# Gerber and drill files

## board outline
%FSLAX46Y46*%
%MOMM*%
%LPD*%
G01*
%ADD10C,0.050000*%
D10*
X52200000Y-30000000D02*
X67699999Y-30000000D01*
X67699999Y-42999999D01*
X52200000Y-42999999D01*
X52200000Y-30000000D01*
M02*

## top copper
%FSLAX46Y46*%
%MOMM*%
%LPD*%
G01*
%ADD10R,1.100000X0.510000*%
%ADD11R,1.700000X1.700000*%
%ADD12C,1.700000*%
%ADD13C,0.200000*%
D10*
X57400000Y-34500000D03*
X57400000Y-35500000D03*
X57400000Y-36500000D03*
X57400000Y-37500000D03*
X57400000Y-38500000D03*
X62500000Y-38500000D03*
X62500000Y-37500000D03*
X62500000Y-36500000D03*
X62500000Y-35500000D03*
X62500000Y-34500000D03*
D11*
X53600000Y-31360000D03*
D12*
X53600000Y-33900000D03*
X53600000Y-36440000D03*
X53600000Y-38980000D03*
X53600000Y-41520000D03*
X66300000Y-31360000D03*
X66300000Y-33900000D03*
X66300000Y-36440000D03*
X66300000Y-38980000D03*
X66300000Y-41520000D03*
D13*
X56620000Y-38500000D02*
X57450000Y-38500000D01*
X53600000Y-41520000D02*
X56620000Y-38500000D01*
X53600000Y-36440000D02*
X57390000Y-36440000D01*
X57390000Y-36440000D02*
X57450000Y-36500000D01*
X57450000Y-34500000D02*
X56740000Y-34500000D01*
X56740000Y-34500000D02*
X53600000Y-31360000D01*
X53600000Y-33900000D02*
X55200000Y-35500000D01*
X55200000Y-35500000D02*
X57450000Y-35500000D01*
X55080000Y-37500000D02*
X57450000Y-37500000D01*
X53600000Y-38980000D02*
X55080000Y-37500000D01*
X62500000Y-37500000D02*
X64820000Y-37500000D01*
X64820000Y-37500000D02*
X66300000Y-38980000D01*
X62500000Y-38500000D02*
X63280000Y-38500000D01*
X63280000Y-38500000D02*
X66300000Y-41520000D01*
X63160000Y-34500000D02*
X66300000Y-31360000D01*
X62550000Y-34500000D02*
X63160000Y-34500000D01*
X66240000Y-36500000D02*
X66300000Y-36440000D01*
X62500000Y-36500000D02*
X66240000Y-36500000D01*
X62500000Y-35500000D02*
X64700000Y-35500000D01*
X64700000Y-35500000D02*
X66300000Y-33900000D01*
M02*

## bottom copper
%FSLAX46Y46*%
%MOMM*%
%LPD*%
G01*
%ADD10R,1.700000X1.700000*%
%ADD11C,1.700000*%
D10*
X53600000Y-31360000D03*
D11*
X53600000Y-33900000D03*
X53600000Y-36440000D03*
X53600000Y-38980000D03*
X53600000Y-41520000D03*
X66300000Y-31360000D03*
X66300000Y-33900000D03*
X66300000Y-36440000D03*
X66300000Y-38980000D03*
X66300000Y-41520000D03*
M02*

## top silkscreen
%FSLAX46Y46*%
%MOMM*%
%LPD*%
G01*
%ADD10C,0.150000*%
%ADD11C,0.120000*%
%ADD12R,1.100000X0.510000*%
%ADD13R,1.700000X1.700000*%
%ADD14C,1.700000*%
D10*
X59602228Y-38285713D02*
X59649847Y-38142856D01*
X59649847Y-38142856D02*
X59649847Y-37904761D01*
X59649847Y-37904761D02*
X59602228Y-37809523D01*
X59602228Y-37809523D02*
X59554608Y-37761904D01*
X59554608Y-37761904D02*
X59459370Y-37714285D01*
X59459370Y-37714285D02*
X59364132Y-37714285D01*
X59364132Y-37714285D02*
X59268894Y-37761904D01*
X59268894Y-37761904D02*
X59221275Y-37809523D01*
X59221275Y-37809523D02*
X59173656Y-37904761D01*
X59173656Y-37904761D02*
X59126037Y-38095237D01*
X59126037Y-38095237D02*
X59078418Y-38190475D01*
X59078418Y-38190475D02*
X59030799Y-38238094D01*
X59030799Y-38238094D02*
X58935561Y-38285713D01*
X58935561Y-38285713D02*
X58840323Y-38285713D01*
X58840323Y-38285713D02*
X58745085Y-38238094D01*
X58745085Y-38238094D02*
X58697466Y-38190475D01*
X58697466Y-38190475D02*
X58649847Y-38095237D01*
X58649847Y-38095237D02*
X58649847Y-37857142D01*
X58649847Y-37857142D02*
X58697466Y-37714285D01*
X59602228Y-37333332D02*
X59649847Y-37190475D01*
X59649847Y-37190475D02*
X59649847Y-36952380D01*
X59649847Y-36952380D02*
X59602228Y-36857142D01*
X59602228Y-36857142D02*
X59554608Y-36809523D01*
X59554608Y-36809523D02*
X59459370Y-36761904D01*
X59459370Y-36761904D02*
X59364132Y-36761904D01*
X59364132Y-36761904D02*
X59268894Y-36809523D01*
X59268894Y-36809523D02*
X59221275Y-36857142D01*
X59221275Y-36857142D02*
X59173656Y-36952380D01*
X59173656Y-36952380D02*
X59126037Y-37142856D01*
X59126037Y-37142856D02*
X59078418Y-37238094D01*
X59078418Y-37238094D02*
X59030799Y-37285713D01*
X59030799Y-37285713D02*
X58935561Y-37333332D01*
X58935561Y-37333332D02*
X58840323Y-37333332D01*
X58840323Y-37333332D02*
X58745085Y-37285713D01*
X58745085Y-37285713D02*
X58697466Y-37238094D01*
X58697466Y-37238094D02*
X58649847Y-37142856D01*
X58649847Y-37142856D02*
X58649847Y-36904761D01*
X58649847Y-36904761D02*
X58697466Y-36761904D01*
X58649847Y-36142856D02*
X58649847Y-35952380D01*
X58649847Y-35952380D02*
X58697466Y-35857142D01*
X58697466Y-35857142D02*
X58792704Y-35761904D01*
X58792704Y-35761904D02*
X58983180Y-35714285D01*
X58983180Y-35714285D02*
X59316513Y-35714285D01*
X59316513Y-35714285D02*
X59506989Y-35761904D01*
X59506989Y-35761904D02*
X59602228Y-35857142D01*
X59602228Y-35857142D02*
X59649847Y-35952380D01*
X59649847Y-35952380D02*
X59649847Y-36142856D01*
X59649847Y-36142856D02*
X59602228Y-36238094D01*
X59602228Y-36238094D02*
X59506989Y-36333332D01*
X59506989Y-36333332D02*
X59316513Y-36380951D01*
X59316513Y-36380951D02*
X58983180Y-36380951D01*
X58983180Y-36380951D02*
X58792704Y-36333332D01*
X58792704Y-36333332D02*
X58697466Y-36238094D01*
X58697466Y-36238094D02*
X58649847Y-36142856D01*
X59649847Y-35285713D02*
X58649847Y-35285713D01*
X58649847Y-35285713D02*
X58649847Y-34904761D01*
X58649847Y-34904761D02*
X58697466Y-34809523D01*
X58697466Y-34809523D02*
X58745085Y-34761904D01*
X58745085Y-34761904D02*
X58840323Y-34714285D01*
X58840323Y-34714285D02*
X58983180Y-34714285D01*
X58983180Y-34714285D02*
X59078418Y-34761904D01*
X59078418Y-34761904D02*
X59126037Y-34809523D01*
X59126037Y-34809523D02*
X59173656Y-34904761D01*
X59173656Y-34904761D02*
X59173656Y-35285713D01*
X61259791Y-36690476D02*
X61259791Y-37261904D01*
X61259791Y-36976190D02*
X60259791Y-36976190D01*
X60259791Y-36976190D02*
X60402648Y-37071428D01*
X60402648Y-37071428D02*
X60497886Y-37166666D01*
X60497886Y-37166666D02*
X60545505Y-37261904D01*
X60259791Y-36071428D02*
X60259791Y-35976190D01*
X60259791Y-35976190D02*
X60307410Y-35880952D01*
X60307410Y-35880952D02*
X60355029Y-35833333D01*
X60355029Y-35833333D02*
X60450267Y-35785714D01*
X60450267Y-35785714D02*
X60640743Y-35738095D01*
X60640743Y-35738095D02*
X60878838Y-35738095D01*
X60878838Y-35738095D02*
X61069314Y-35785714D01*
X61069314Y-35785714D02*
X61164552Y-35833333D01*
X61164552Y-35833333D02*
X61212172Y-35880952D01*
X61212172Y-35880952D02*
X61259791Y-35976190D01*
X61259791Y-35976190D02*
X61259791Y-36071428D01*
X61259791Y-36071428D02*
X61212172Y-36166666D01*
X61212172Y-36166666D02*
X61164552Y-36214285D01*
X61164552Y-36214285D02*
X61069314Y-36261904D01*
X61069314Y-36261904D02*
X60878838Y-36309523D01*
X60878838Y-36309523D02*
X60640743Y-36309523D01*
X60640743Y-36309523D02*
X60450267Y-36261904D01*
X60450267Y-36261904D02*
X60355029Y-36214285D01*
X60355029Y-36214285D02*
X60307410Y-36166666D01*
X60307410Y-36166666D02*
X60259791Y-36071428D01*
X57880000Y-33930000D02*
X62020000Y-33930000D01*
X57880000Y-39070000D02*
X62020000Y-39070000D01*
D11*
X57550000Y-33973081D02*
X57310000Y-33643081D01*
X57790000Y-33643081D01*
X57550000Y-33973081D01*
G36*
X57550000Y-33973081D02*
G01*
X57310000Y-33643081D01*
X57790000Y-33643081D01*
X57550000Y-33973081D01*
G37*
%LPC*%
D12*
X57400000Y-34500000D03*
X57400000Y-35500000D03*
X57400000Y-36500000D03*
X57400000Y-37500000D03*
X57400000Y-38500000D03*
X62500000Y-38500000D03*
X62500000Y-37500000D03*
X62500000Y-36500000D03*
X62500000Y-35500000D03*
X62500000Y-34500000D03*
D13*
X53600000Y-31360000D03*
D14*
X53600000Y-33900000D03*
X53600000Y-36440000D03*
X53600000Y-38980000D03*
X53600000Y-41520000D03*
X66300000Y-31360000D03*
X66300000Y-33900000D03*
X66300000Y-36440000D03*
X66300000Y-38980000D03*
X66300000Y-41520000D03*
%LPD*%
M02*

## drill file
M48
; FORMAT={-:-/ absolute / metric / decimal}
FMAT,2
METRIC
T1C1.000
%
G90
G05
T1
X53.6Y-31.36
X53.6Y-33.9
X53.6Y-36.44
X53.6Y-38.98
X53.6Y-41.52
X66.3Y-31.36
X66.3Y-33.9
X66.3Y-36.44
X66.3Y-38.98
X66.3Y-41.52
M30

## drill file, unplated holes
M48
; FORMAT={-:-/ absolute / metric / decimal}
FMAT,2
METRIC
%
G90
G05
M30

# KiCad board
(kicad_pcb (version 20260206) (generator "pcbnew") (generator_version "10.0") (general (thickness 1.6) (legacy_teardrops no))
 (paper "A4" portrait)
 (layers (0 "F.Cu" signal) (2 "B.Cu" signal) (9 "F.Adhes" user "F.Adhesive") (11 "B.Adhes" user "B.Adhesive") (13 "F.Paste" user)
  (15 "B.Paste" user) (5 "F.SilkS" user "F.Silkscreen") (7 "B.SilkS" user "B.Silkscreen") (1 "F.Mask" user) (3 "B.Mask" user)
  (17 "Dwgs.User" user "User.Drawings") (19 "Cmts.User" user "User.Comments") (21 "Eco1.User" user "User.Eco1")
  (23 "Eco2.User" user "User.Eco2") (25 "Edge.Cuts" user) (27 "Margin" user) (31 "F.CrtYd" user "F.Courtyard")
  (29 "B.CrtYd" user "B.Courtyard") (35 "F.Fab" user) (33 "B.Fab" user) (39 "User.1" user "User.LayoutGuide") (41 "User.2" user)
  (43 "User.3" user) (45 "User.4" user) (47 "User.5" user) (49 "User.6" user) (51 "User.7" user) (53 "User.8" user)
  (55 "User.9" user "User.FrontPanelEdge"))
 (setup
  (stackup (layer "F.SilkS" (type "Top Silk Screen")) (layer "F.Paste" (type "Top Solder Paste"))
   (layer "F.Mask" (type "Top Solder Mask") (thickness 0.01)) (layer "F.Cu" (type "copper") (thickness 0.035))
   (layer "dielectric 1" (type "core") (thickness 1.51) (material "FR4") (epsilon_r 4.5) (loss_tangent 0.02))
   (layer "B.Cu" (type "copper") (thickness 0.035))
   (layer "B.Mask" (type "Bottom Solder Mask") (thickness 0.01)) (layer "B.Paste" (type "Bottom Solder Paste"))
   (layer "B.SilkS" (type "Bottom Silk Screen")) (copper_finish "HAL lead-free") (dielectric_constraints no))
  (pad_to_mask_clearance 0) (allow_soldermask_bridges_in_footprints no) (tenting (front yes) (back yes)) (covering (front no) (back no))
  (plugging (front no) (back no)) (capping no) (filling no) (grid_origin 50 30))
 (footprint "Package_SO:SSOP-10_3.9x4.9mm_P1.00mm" (layer "F.Cu") (at 59.95 36.5)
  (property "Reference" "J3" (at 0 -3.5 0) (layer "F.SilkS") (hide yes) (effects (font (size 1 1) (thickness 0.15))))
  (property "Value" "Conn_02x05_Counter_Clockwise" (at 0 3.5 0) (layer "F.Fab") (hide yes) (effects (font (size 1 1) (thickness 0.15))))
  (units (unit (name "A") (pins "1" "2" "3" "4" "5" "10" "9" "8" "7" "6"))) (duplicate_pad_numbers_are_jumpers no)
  (fp_line (start -2.07 -2.57) (end 2.07 -2.57) (stroke (width 0.15) (type solid)) (layer "F.SilkS"))
  (fp_line (start -2.07 2.57) (end 2.07 2.57) (stroke (width 0.15) (type solid)) (layer "F.SilkS"))
  (fp_poly
   (pts (xy -2.4 -2.526919) (xy -2.64 -2.856919) (xy -2.16 -2.856919) (xy -2.4 -2.526919)) (stroke (width 0.12) (type solid)) (fill yes)
   (layer "F.SilkS"))
  (pad "1" smd rect (at -2.55 -2) (size 1.1 0.51) (layers "F.Cu" "F.Mask" "F.Paste") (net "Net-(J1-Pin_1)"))
  (pad "2" smd rect (at -2.55 -1) (size 1.1 0.51) (layers "F.Cu" "F.Mask" "F.Paste") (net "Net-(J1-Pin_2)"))
  (pad "3" smd rect (at -2.55 0) (size 1.1 0.51) (layers "F.Cu" "F.Mask" "F.Paste") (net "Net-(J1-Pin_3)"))
  (pad "4" smd rect (at -2.55 1) (size 1.1 0.51) (layers "F.Cu" "F.Mask" "F.Paste") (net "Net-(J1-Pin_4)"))
  (pad "5" smd rect (at -2.55 2) (size 1.1 0.51) (layers "F.Cu" "F.Mask" "F.Paste") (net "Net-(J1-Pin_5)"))
  (pad "6" smd rect (at 2.55 2) (size 1.1 0.51) (layers "F.Cu" "F.Mask" "F.Paste") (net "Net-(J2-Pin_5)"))
  (pad "7" smd rect (at 2.55 1) (size 1.1 0.51) (layers "F.Cu" "F.Mask" "F.Paste") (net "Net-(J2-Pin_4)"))
  (pad "8" smd rect (at 2.55 0) (size 1.1 0.51) (layers "F.Cu" "F.Mask" "F.Paste") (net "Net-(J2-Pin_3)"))
  (pad "9" smd rect (at 2.55 -1) (size 1.1 0.51) (layers "F.Cu" "F.Mask" "F.Paste") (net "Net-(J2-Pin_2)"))
  (pad "10" smd rect (at 2.55 -2) (size 1.1 0.51) (layers "F.Cu" "F.Mask" "F.Paste") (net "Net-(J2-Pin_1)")))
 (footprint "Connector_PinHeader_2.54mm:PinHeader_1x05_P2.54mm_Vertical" (layer "B.Cu") (at 53.6 31.36 180)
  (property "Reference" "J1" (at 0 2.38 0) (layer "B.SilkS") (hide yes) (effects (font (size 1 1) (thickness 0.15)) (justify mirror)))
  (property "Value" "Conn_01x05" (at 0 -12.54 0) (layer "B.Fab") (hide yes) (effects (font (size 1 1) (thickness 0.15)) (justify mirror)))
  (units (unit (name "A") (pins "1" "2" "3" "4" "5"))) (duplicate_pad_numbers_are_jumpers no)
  (pad "1" thru_hole rect (at 0 0 180) (size 1.7 1.7) (drill 1) (layers "*.Cu" "*.Mask") (remove_unused_layers no) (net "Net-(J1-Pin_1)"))
  (pad "2" thru_hole circle (at 0 -2.54 180) (size 1.7 1.7) (drill 1) (layers "*.Cu" "*.Mask") (remove_unused_layers no)
   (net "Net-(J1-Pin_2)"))
  (pad "3" thru_hole circle (at 0 -5.08 180) (size 1.7 1.7) (drill 1) (layers "*.Cu" "*.Mask") (remove_unused_layers no)
   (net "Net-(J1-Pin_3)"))
  (pad "4" thru_hole circle (at 0 -7.62 180) (size 1.7 1.7) (drill 1) (layers "*.Cu" "*.Mask") (remove_unused_layers no)
   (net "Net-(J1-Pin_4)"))
  (pad "5" thru_hole circle (at 0 -10.16 180) (size 1.7 1.7) (drill 1) (layers "*.Cu" "*.Mask") (remove_unused_layers no)
   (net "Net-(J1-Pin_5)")))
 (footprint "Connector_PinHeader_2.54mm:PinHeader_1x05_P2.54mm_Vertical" (layer "B.Cu") (at 66.3 31.36 180)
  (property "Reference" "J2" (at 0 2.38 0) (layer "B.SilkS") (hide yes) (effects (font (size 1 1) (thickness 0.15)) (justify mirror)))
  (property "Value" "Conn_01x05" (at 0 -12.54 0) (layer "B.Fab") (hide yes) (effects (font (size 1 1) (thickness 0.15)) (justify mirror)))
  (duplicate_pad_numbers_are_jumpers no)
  (pad "1" thru_hole circle (at 0 0 180) (size 1.7 1.7) (drill 1) (layers "*.Cu" "*.Mask") (remove_unused_layers no) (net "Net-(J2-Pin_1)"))
  (pad "2" thru_hole circle (at 0 -2.54 180) (size 1.7 1.7) (drill 1) (layers "*.Cu" "*.Mask") (remove_unused_layers no)
   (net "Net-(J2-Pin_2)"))
  (pad "3" thru_hole circle (at 0 -5.08 180) (size 1.7 1.7) (drill 1) (layers "*.Cu" "*.Mask") (remove_unused_layers no)
   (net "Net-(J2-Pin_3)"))
  (pad "4" thru_hole circle (at 0 -7.62 180) (size 1.7 1.7) (drill 1) (layers "*.Cu" "*.Mask") (remove_unused_layers no)
   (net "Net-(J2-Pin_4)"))
  (pad "5" thru_hole circle (at 0 -10.16 180) (size 1.7 1.7) (drill 1) (layers "*.Cu" "*.Mask") (remove_unused_layers no)
   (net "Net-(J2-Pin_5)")))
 (gr_rect (start 52.2 30) (end 67.699999 42.999999) (stroke (width 0.05) (type default)) (fill no) (layer "Edge.Cuts"))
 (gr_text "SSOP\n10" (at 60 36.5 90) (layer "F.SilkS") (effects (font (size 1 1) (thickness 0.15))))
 (segment (start 57.45 34.5) (end 56.74 34.5) (width 0.2) (layer "F.Cu") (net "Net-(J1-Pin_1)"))
 (segment (start 56.74 34.5) (end 53.6 31.36) (width 0.2) (layer "F.Cu") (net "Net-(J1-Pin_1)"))
 (segment (start 53.6 33.9) (end 55.2 35.5) (width 0.2) (layer "F.Cu") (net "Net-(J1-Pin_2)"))
 (segment (start 55.2 35.5) (end 57.45 35.5) (width 0.2) (layer "F.Cu") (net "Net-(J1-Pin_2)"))
 (segment (start 53.6 36.44) (end 57.39 36.44) (width 0.2) (layer "F.Cu") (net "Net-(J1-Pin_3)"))
 (segment (start 57.39 36.44) (end 57.45 36.5) (width 0.2) (layer "F.Cu") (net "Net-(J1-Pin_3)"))
 (segment (start 55.08 37.5) (end 57.45 37.5) (width 0.2) (layer "F.Cu") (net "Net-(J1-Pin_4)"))
 (segment (start 53.6 38.98) (end 55.08 37.5) (width 0.2) (layer "F.Cu") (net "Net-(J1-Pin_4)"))
 (segment (start 56.62 38.5) (end 57.45 38.5) (width 0.2) (layer "F.Cu") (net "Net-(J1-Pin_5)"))
 (segment (start 53.6 41.52) (end 56.62 38.5) (width 0.2) (layer "F.Cu") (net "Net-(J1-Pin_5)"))
 (segment (start 62.5 38.5) (end 63.28 38.5) (width 0.2) (layer "F.Cu") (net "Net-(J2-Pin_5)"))
 (segment (start 63.28 38.5) (end 66.3 41.52) (width 0.2) (layer "F.Cu") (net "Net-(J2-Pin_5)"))
 (segment (start 62.5 37.5) (end 64.82 37.5) (width 0.2) (layer "F.Cu") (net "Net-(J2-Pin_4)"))
 (segment (start 64.82 37.5) (end 66.3 38.98) (width 0.2) (layer "F.Cu") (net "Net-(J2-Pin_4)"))
 (segment (start 66.24 36.5) (end 66.3 36.44) (width 0.2) (layer "F.Cu") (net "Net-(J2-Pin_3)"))
 (segment (start 62.5 36.5) (end 66.24 36.5) (width 0.2) (layer "F.Cu") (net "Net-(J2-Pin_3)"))
 (segment (start 62.5 35.5) (end 64.7 35.5) (width 0.2) (layer "F.Cu") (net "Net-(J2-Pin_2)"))
 (segment (start 64.7 35.5) (end 66.3 33.9) (width 0.2) (layer "F.Cu") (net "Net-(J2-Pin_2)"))
 (segment (start 63.16 34.5) (end 66.3 31.36) (width 0.2) (layer "F.Cu") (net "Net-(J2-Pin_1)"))
 (segment (start 62.55 34.5) (end 63.16 34.5) (width 0.2) (layer "F.Cu") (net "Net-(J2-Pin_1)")))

